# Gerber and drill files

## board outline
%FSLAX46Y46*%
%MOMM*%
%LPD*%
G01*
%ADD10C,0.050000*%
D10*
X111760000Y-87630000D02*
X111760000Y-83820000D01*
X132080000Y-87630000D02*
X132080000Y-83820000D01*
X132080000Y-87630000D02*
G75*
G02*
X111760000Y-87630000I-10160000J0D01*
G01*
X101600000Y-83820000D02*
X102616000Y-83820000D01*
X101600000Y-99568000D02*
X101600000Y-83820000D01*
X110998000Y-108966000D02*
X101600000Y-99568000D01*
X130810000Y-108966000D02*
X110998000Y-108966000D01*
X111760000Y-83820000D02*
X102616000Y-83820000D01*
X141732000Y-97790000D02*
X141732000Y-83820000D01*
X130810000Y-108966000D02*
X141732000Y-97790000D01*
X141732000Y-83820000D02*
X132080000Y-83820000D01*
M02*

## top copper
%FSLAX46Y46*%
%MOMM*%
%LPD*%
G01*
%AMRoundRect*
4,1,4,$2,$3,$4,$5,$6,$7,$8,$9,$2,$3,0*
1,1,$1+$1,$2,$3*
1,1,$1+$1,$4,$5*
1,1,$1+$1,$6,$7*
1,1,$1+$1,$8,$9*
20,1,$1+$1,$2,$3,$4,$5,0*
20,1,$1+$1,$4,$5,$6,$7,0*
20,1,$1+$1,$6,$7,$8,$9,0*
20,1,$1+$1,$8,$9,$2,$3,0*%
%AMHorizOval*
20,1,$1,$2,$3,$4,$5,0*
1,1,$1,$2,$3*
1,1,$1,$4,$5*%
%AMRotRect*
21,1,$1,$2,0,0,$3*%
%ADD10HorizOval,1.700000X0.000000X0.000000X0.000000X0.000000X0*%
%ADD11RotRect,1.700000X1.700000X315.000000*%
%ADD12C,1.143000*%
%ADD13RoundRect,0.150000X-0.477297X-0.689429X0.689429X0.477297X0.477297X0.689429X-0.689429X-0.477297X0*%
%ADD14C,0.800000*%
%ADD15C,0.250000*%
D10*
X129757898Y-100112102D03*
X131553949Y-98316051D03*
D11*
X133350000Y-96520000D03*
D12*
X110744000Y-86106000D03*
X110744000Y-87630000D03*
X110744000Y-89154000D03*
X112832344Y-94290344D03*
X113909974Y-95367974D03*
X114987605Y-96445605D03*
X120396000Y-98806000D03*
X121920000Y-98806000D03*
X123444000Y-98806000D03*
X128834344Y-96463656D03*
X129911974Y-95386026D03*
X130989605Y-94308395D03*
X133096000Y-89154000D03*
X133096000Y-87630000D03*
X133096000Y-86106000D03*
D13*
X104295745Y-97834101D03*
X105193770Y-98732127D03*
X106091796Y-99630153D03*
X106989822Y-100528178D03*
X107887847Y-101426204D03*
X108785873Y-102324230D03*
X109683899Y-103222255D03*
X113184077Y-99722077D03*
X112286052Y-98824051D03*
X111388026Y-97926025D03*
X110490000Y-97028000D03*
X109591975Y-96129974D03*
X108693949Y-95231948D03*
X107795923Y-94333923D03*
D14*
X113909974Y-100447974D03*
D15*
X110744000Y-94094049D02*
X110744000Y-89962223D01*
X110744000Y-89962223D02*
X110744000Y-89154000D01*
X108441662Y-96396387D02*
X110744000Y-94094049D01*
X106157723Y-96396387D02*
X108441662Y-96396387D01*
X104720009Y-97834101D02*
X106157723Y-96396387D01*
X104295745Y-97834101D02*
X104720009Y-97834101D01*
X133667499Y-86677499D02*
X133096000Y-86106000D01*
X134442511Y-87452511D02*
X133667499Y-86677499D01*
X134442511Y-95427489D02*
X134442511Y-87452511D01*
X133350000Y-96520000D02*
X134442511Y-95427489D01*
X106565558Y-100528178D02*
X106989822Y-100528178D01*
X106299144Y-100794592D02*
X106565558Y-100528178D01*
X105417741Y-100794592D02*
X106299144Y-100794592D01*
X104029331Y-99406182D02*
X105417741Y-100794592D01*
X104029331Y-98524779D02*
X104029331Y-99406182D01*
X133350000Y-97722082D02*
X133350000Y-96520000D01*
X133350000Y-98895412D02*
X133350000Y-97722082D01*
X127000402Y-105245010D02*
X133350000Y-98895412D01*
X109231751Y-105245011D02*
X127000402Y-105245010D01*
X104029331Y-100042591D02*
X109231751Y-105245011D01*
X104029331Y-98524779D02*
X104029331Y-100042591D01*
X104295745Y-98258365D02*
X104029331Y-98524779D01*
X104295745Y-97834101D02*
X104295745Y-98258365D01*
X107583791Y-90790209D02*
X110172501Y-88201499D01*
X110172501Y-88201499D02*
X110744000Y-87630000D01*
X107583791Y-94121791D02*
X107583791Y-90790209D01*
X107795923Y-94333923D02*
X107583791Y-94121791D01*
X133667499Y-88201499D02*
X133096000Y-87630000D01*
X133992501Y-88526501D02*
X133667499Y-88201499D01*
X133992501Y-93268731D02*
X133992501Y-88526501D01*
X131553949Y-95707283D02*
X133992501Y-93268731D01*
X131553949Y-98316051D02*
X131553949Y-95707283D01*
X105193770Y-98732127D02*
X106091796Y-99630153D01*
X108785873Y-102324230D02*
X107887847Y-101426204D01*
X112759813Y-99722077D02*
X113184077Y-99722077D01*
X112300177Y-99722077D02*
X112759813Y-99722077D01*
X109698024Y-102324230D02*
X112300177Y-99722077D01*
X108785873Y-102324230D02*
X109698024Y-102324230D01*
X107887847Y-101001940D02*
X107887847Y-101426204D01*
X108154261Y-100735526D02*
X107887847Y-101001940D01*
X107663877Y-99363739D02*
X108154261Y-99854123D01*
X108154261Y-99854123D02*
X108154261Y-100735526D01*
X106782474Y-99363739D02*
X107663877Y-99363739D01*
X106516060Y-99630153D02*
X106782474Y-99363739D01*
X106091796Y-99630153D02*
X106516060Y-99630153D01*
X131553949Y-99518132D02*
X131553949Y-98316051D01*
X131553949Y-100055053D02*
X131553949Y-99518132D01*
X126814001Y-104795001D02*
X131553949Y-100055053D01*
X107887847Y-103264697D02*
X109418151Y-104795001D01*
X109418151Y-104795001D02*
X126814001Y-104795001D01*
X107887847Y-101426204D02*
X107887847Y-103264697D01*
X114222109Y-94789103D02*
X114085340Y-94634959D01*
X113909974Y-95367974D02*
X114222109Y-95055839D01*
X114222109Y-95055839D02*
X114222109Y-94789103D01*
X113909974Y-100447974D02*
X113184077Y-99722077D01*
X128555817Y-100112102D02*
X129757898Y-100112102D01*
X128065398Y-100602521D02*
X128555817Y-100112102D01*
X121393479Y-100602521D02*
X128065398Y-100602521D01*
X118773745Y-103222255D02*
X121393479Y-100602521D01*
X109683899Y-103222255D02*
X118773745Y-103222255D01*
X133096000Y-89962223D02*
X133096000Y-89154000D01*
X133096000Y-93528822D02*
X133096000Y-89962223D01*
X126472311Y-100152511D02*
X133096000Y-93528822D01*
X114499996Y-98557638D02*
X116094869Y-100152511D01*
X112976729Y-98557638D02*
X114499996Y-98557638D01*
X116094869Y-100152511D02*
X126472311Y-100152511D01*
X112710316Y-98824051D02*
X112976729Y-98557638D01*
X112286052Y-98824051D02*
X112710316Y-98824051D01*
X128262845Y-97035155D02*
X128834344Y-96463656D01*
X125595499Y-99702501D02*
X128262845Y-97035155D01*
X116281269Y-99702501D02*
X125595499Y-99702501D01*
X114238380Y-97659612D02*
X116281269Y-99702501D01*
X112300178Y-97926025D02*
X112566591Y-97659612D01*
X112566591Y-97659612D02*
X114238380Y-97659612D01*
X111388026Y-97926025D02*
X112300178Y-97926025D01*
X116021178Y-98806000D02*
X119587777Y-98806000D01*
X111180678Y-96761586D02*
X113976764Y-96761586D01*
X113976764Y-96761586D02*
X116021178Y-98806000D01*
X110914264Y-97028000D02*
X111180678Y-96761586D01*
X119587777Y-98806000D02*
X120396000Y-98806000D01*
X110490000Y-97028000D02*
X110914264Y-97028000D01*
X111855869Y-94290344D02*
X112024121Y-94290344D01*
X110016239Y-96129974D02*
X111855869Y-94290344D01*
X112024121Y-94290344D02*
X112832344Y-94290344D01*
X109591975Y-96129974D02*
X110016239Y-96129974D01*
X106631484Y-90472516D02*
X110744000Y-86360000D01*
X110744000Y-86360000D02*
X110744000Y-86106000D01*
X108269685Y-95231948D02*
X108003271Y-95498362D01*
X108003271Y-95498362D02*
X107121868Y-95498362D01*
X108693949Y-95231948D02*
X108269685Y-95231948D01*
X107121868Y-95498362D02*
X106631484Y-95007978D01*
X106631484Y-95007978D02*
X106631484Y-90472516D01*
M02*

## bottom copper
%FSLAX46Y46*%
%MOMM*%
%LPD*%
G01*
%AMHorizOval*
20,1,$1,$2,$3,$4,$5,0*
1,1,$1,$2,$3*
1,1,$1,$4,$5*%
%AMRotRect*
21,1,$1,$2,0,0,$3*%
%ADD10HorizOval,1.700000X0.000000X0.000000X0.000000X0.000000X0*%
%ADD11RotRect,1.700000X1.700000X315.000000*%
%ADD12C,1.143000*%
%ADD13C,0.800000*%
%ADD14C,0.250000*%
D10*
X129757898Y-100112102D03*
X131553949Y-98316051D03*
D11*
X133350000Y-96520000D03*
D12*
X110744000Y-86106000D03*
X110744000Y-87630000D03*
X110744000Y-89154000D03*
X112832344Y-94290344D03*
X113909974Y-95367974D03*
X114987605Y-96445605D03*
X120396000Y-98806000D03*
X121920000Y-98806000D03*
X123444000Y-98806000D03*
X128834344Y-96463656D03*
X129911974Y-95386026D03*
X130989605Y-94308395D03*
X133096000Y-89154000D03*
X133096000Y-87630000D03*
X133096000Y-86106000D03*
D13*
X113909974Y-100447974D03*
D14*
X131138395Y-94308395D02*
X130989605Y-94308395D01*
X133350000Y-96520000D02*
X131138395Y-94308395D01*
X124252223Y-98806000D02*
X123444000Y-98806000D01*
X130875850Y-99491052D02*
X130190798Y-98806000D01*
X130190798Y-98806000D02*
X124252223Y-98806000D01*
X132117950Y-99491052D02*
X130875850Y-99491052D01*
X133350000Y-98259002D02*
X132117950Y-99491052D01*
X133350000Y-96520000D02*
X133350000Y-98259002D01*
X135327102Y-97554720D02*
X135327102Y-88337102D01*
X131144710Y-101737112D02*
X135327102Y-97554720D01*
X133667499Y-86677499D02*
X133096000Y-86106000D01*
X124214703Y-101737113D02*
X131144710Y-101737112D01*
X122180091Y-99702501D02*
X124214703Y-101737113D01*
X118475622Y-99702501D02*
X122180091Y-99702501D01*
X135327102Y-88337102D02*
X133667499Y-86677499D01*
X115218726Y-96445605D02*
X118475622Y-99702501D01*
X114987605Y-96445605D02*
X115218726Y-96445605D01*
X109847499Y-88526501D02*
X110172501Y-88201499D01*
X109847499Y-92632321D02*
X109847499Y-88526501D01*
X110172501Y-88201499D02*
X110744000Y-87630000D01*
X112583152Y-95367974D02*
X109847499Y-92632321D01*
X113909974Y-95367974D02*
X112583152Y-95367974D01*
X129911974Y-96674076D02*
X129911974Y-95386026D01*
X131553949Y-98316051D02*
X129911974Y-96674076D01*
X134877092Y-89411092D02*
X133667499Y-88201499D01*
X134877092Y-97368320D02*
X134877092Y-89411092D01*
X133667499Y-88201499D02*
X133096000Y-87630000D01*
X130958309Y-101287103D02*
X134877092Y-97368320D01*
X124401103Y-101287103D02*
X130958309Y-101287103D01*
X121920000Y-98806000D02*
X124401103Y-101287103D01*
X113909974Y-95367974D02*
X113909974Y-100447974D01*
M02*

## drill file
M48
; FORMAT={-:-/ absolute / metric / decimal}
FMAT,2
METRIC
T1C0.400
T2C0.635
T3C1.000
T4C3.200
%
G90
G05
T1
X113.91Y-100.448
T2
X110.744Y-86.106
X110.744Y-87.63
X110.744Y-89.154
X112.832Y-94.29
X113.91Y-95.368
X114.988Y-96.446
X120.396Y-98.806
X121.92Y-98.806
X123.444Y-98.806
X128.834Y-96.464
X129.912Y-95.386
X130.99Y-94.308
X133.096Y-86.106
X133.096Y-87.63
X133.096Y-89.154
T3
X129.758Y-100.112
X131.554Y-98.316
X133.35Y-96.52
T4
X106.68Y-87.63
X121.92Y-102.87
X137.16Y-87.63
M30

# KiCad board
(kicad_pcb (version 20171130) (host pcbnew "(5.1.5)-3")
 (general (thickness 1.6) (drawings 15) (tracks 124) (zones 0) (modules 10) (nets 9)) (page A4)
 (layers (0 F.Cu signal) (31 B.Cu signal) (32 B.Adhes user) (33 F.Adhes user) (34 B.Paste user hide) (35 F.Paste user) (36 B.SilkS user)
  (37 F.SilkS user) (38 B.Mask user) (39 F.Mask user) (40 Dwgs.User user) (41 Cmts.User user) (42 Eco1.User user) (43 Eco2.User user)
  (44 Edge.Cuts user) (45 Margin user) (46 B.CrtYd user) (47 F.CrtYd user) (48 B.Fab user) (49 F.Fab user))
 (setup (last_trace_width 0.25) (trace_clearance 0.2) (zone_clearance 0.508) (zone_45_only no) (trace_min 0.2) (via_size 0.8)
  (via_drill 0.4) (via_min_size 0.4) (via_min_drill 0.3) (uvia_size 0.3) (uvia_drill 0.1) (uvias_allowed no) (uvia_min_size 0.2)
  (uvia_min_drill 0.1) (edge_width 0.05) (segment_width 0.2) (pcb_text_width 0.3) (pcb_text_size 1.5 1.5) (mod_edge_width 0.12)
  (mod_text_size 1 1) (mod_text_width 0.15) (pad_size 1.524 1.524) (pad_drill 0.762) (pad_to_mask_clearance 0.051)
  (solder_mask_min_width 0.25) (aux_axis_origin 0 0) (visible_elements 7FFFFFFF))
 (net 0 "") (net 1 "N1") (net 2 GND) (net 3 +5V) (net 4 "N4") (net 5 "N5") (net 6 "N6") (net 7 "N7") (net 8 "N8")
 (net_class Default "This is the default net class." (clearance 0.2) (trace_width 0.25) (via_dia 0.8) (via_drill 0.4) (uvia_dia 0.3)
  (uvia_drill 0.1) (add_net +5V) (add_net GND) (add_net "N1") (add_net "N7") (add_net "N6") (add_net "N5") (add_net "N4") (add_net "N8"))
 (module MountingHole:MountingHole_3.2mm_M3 (layer F.Cu) (at 121.92 102.87)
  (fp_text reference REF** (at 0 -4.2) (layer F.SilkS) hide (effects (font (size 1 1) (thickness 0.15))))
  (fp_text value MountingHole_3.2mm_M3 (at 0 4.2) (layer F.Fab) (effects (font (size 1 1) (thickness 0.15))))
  (pad 1 np_thru_hole circle (at 0 0) (size 3.2 3.2) (drill 3.2) (layers *.Cu *.Mask)))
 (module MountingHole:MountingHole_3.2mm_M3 (layer F.Cu) (at 137.16 87.63)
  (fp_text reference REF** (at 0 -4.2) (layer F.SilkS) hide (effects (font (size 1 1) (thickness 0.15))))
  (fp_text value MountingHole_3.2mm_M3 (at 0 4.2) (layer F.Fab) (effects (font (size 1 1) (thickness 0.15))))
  (pad 1 np_thru_hole circle (at 0 0) (size 3.2 3.2) (drill 3.2) (layers *.Cu *.Mask)))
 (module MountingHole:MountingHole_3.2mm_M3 (layer F.Cu) (at 106.68 87.63)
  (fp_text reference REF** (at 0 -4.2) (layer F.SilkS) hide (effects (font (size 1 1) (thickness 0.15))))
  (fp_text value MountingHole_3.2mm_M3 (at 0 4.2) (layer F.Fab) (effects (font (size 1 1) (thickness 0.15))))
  (pad 1 np_thru_hole circle (at 0 0) (size 3.2 3.2) (drill 3.2) (layers *.Cu *.Mask)))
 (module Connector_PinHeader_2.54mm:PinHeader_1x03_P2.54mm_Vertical (layer F.Cu) (at 133.35 96.52 315)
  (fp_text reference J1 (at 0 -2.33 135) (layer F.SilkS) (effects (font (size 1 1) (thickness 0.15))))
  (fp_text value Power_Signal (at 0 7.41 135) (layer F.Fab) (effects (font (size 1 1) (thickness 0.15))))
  (pad 3 thru_hole oval (at 0 5.08 315) (size 1.7 1.7) (drill 1) (layers *.Cu *.Mask) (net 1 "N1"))
  (pad 2 thru_hole oval (at 0 2.54 315) (size 1.7 1.7) (drill 1) (layers *.Cu *.Mask) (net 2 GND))
  (pad 1 thru_hole rect (at 0 0 315) (size 1.7 1.7) (drill 1) (layers *.Cu *.Mask) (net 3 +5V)))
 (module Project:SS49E (layer F.Cu) (at 110.744 88.9 90)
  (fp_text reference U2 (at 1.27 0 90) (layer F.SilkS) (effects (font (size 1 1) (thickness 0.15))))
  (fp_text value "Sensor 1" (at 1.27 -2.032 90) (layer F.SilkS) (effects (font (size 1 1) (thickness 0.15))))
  (pad 3 thru_hole circle (at 2.794 0 90) (size 1.143 1.143) (drill 0.635) (layers *.Cu *.Mask) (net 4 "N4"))
  (pad 2 thru_hole circle (at 1.27 0 90) (size 1.143 1.143) (drill 0.635) (layers *.Cu *.Mask) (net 2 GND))
  (pad 1 thru_hole circle (at -0.254 0 90) (size 1.143 1.143) (drill 0.635) (layers *.Cu *.Mask) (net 3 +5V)))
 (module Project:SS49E (layer F.Cu) (at 114.808 96.266 135)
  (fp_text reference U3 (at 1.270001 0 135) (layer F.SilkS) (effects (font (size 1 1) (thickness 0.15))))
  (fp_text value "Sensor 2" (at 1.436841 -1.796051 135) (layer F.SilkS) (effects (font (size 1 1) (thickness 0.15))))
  (pad 3 thru_hole circle (at 2.794 0 135) (size 1.143 1.143) (drill 0.635) (layers *.Cu *.Mask) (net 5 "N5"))
  (pad 2 thru_hole circle (at 1.27 0 135) (size 1.143 1.143) (drill 0.635) (layers *.Cu *.Mask) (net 2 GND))
  (pad 1 thru_hole circle (at -0.254 0 135) (size 1.143 1.143) (drill 0.635) (layers *.Cu *.Mask) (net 3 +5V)))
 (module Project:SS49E (layer F.Cu) (at 123.19 98.806 180)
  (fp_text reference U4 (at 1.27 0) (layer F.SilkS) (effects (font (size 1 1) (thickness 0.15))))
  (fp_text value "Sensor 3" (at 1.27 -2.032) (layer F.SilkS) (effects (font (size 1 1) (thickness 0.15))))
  (pad 3 thru_hole circle (at 2.794 0 180) (size 1.143 1.143) (drill 0.635) (layers *.Cu *.Mask) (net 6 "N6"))
  (pad 2 thru_hole circle (at 1.27 0 180) (size 1.143 1.143) (drill 0.635) (layers *.Cu *.Mask) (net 2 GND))
  (pad 1 thru_hole circle (at -0.254 0 180) (size 1.143 1.143) (drill 0.635) (layers *.Cu *.Mask) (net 3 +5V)))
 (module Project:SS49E (layer F.Cu) (at 130.81 94.488 225)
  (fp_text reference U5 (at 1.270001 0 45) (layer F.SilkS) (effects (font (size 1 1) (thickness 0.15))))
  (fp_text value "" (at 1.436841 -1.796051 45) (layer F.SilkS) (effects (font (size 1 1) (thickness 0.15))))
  (pad 3 thru_hole circle (at 2.794 0 225) (size 1.143 1.143) (drill 0.635) (layers *.Cu *.Mask) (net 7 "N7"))
  (pad 2 thru_hole circle (at 1.27 0 225) (size 1.143 1.143) (drill 0.635) (layers *.Cu *.Mask) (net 2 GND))
  (pad 1 thru_hole circle (at -0.254 0 225) (size 1.143 1.143) (drill 0.635) (layers *.Cu *.Mask) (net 3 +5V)))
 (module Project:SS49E (layer F.Cu) (at 133.096 86.36 270)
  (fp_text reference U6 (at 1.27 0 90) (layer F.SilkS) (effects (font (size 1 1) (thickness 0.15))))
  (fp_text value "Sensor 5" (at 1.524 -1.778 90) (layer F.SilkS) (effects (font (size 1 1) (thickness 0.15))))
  (pad 3 thru_hole circle (at 2.794 0 270) (size 1.143 1.143) (drill 0.635) (layers *.Cu *.Mask) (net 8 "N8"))
  (pad 2 thru_hole circle (at 1.27 0 270) (size 1.143 1.143) (drill 0.635) (layers *.Cu *.Mask) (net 2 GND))
  (pad 1 thru_hole circle (at -0.254 0 270) (size 1.143 1.143) (drill 0.635) (layers *.Cu *.Mask) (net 3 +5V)))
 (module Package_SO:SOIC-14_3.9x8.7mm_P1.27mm (layer F.Cu) (at 108.739911 98.778089 45)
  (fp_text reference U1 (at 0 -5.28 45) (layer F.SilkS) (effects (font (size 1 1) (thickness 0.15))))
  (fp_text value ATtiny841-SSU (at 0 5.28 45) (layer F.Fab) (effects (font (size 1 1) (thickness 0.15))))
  (pad 1 smd roundrect (at -2.475 -3.81 45) (size 1.95 0.6) (layers F.Cu F.Paste F.Mask) (roundrect_rratio 0.25) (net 3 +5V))
  (pad 2 smd roundrect (at -2.475 -2.54 45) (size 1.95 0.6) (layers F.Cu F.Paste F.Mask) (roundrect_rratio 0.25) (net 2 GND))
  (pad 3 smd roundrect (at -2.475 -1.27 45) (size 1.95 0.6) (layers F.Cu F.Paste F.Mask) (roundrect_rratio 0.25) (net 2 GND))
  (pad 4 smd roundrect (at -2.475 0 45) (size 1.95 0.6) (layers F.Cu F.Paste F.Mask) (roundrect_rratio 0.25) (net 3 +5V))
  (pad 5 smd roundrect (at -2.475 1.27 45) (size 1.95 0.6) (layers F.Cu F.Paste F.Mask) (roundrect_rratio 0.25) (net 2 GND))
  (pad 6 smd roundrect (at -2.475 2.54 45) (size 1.95 0.6) (layers F.Cu F.Paste F.Mask) (roundrect_rratio 0.25) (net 2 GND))
  (pad 7 smd roundrect (at -2.475 3.81 45) (size 1.95 0.6) (layers F.Cu F.Paste F.Mask) (roundrect_rratio 0.25) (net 1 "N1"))
  (pad 8 smd roundrect (at 2.475 3.81 45) (size 1.95 0.6) (layers F.Cu F.Paste F.Mask) (roundrect_rratio 0.25) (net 2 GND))
  (pad 9 smd roundrect (at 2.475 2.54 45) (size 1.95 0.6) (layers F.Cu F.Paste F.Mask) (roundrect_rratio 0.25) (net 8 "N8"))
  (pad 10 smd roundrect (at 2.475 1.27 45) (size 1.95 0.6) (layers F.Cu F.Paste F.Mask) (roundrect_rratio 0.25) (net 7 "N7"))
  (pad 11 smd roundrect (at 2.475 0 45) (size 1.95 0.6) (layers F.Cu F.Paste F.Mask) (roundrect_rratio 0.25) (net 6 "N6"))
  (pad 12 smd roundrect (at 2.475 -1.27 45) (size 1.95 0.6) (layers F.Cu F.Paste F.Mask) (roundrect_rratio 0.25) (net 5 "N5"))
  (pad 13 smd roundrect (at 2.475 -2.54 45) (size 1.95 0.6) (layers F.Cu F.Paste F.Mask) (roundrect_rratio 0.25) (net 4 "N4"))
  (pad 14 smd roundrect (at 2.475 -3.81 45) (size 1.95 0.6) (layers F.Cu F.Paste F.Mask) (roundrect_rratio 0.25) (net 2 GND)))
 (gr_line (start 111.76 87.63) (end 111.76 83.82) (layer Edge.Cuts) (width 0.05))
 (gr_line (start 132.08 87.63) (end 132.08 83.82) (layer Edge.Cuts) (width 0.05))
 (gr_arc (start 121.92 87.63) (end 111.76 87.63) (angle -180) (layer Edge.Cuts) (width 0.05))
 (gr_line (start 101.6 83.82) (end 102.616 83.82) (layer Edge.Cuts) (width 0.05))
 (gr_line (start 101.6 99.568) (end 101.6 83.82) (layer Edge.Cuts) (width 0.05))
 (gr_line (start 110.998 108.966) (end 101.6 99.568) (layer Edge.Cuts) (width 0.05))
 (gr_line (start 130.81 108.966) (end 110.998 108.966) (layer Edge.Cuts) (width 0.05))
 (gr_line (start 111.76 83.82) (end 102.616 83.82) (layer Edge.Cuts) (width 0.05))
 (gr_line (start 141.732 97.79) (end 141.732 83.82) (layer Edge.Cuts) (width 0.05))
 (gr_line (start 130.81 108.966) (end 141.732 97.79) (layer Edge.Cuts) (width 0.05))
 (gr_line (start 141.732 83.82) (end 132.08 83.82) (layer Edge.Cuts) (width 0.05))
 (segment (start 110.744 94.094049) (end 110.744 89.962223) (width 0.25) (layer F.Cu) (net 3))
 (segment (start 110.744 89.962223) (end 110.744 89.154) (width 0.25) (layer F.Cu) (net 3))
 (segment (start 108.441662 96.396387) (end 110.744 94.094049) (width 0.25) (layer F.Cu) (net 3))
 (segment (start 106.157723 96.396387) (end 108.441662 96.396387) (width 0.25) (layer F.Cu) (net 3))
 (segment (start 104.720009 97.834101) (end 106.157723 96.396387) (width 0.25) (layer F.Cu) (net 3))
 (segment (start 104.295745 97.834101) (end 104.720009 97.834101) (width 0.25) (layer F.Cu) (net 3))
 (segment (start 133.667499 86.677499) (end 133.096 86.106) (width 0.25) (layer F.Cu) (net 3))
 (segment (start 134.442511 87.452511) (end 133.667499 86.677499) (width 0.25) (layer F.Cu) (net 3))
 (segment (start 134.442511 95.427489) (end 134.442511 87.452511) (width 0.25) (layer F.Cu) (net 3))
 (segment (start 133.35 96.52) (end 134.442511 95.427489) (width 0.25) (layer F.Cu) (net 3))
 (segment (start 106.565558 100.528178) (end 106.989822 100.528178) (width 0.25) (layer F.Cu) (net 3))
 (segment (start 106.299144 100.794592) (end 106.565558 100.528178) (width 0.25) (layer F.Cu) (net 3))
 (segment (start 105.417741 100.794592) (end 106.299144 100.794592) (width 0.25) (layer F.Cu) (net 3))
 (segment (start 104.029331 99.406182) (end 105.417741 100.794592) (width 0.25) (layer F.Cu) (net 3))
 (segment (start 104.029331 98.524779) (end 104.029331 99.406182) (width 0.25) (layer F.Cu) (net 3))
 (segment (start 131.138395 94.308395) (end 130.989605 94.308395) (width 0.25) (layer B.Cu) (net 3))
 (segment (start 133.35 96.52) (end 131.138395 94.308395) (width 0.25) (layer B.Cu) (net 3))
 (segment (start 124.252223 98.806) (end 123.444 98.806) (width 0.25) (layer B.Cu) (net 3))
 (segment (start 130.87585 99.491052) (end 130.190798 98.806) (width 0.25) (layer B.Cu) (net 3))
 (segment (start 130.190798 98.806) (end 124.252223 98.806) (width 0.25) (layer B.Cu) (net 3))
 (segment (start 132.11795 99.491052) (end 130.87585 99.491052) (width 0.25) (layer B.Cu) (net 3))
 (segment (start 133.35 98.259002) (end 132.11795 99.491052) (width 0.25) (layer B.Cu) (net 3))
 (segment (start 133.35 96.52) (end 133.35 98.259002) (width 0.25) (layer B.Cu) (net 3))
 (segment (start 135.327102 97.55472) (end 135.327102 88.337102) (width 0.25) (layer B.Cu) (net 3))
 (segment (start 131.14471 101.737112) (end 135.327102 97.55472) (width 0.25) (layer B.Cu) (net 3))
 (segment (start 133.667499 86.677499) (end 133.096 86.106) (width 0.25) (layer B.Cu) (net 3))
 (segment (start 124.214703 101.737113) (end 131.14471 101.737112) (width 0.25) (layer B.Cu) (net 3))
 (segment (start 122.180091 99.702501) (end 124.214703 101.737113) (width 0.25) (layer B.Cu) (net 3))
 (segment (start 118.475622 99.702501) (end 122.180091 99.702501) (width 0.25) (layer B.Cu) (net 3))
 (segment (start 135.327102 88.337102) (end 133.667499 86.677499) (width 0.25) (layer B.Cu) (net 3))
 (segment (start 115.218726 96.445605) (end 118.475622 99.702501) (width 0.25) (layer B.Cu) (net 3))
 (segment (start 114.987605 96.445605) (end 115.218726 96.445605) (width 0.25) (layer B.Cu) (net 3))
 (segment (start 133.35 97.722082) (end 133.35 96.52) (width 0.25) (layer F.Cu) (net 3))
 (segment (start 133.35 98.895412) (end 133.35 97.722082) (width 0.25) (layer F.Cu) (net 3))
 (segment (start 127.000402 105.24501) (end 133.35 98.895412) (width 0.25) (layer F.Cu) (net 3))
 (segment (start 109.231751 105.245011) (end 127.000402 105.24501) (width 0.25) (layer F.Cu) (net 3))
 (segment (start 104.029331 100.042591) (end 109.231751 105.245011) (width 0.25) (layer F.Cu) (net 3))
 (segment (start 104.029331 98.524779) (end 104.029331 100.042591) (width 0.25) (layer F.Cu) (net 3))
 (segment (start 104.295745 98.258365) (end 104.029331 98.524779) (width 0.25) (layer F.Cu) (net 3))
 (segment (start 104.295745 97.834101) (end 104.295745 98.258365) (width 0.25) (layer F.Cu) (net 3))
 (segment (start 107.583791 90.790209) (end 110.172501 88.201499) (width 0.25) (layer F.Cu) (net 2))
 (segment (start 110.172501 88.201499) (end 110.744 87.63) (width 0.25) (layer F.Cu) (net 2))
 (segment (start 107.583791 94.121791) (end 107.583791 90.790209) (width 0.25) (layer F.Cu) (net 2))
 (segment (start 107.795923 94.333923) (end 107.583791 94.121791) (width 0.25) (layer F.Cu) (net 2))
 (segment (start 133.667499 88.201499) (end 133.096 87.63) (width 0.25) (layer F.Cu) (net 2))
 (segment (start 133.992501 88.526501) (end 133.667499 88.201499) (width 0.25) (layer F.Cu) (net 2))
 (segment (start 133.992501 93.268731) (end 133.992501 88.526501) (width 0.25) (layer F.Cu) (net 2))
 (segment (start 131.553949 95.707283) (end 133.992501 93.268731) (width 0.25) (layer F.Cu) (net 2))
 (segment (start 131.553949 98.316051) (end 131.553949 95.707283) (width 0.25) (layer F.Cu) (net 2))
 (segment (start 105.19377 98.732127) (end 106.091796 99.630153) (width 0.25) (layer F.Cu) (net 2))
 (segment (start 108.785873 102.32423) (end 107.887847 101.426204) (width 0.25) (layer F.Cu) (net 2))
 (segment (start 112.759813 99.722077) (end 113.184077 99.722077) (width 0.25) (layer F.Cu) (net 2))
 (segment (start 112.300177 99.722077) (end 112.759813 99.722077) (width 0.25) (layer F.Cu) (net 2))
 (segment (start 109.698024 102.32423) (end 112.300177 99.722077) (width 0.25) (layer F.Cu) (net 2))
 (segment (start 108.785873 102.32423) (end 109.698024 102.32423) (width 0.25) (layer F.Cu) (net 2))
 (segment (start 107.887847 101.00194) (end 107.887847 101.426204) (width 0.25) (layer F.Cu) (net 2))
 (segment (start 108.154261 100.735526) (end 107.887847 101.00194) (width 0.25) (layer F.Cu) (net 2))
 (segment (start 107.663877 99.363739) (end 108.154261 99.854123) (width 0.25) (layer F.Cu) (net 2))
 (segment (start 108.154261 99.854123) (end 108.154261 100.735526) (width 0.25) (layer F.Cu) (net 2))
 (segment (start 106.782474 99.363739) (end 107.663877 99.363739) (width 0.25) (layer F.Cu) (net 2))
 (segment (start 106.51606 99.630153) (end 106.782474 99.363739) (width 0.25) (layer F.Cu) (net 2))
 (segment (start 106.091796 99.630153) (end 106.51606 99.630153) (width 0.25) (layer F.Cu) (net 2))
 (segment (start 131.553949 99.518132) (end 131.553949 98.316051) (width 0.25) (layer F.Cu) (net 2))
 (segment (start 131.553949 100.055053) (end 131.553949 99.518132) (width 0.25) (layer F.Cu) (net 2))
 (segment (start 126.814001 104.795001) (end 131.553949 100.055053) (width 0.25) (layer F.Cu) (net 2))
 (segment (start 107.887847 103.264697) (end 109.418151 104.795001) (width 0.25) (layer F.Cu) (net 2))
 (segment (start 109.418151 104.795001) (end 126.814001 104.795001) (width 0.25) (layer F.Cu) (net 2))
 (segment (start 107.887847 101.426204) (end 107.887847 103.264697) (width 0.25) (layer F.Cu) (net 2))
 (segment (start 109.847499 88.526501) (end 110.172501 88.201499) (width 0.25) (layer B.Cu) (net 2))
 (segment (start 109.847499 92.632321) (end 109.847499 88.526501) (width 0.25) (layer B.Cu) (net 2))
 (segment (start 110.172501 88.201499) (end 110.744 87.63) (width 0.25) (layer B.Cu) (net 2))
 (segment (start 112.583152 95.367974) (end 109.847499 92.632321) (width 0.25) (layer B.Cu) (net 2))
 (segment (start 113.909974 95.367974) (end 112.583152 95.367974) (width 0.25) (layer B.Cu) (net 2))
 (segment (start 129.911974 96.674076) (end 129.911974 95.386026) (width 0.25) (layer B.Cu) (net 2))
 (segment (start 131.553949 98.316051) (end 129.911974 96.674076) (width 0.25) (layer B.Cu) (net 2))
 (segment (start 114.222109 94.789103) (end 114.08534 94.634959) (width 0.25) (layer F.Cu) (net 2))
 (segment (start 113.909974 95.367974) (end 114.222109 95.055839) (width 0.25) (layer F.Cu) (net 2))
 (segment (start 114.222109 95.055839) (end 114.222109 94.789103) (width 0.25) (layer F.Cu) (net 2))
 (segment (start 134.877092 89.411092) (end 133.667499 88.201499) (width 0.25) (layer B.Cu) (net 2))
 (segment (start 134.877092 97.36832) (end 134.877092 89.411092) (width 0.25) (layer B.Cu) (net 2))
 (segment (start 133.667499 88.201499) (end 133.096 87.63) (width 0.25) (layer B.Cu) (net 2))
 (segment (start 130.958309 101.287103) (end 134.877092 97.36832) (width 0.25) (layer B.Cu) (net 2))
 (segment (start 124.401103 101.287103) (end 130.958309 101.287103) (width 0.25) (layer B.Cu) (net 2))
 (segment (start 121.92 98.806) (end 124.401103 101.287103) (width 0.25) (layer B.Cu) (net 2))
 (segment (start 113.909974 95.367974) (end 113.909974 100.447974) (width 0.25) (layer B.Cu) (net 2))
 (via (at 113.909974 100.447974) (size 0.8) (drill 0.4) (layers F.Cu B.Cu) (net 2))
 (segment (start 113.909974 100.447974) (end 113.184077 99.722077) (width 0.25) (layer F.Cu) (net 2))
 (segment (start 128.555817 100.112102) (end 129.757898 100.112102) (width 0.25) (layer F.Cu) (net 1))
 (segment (start 128.065398 100.602521) (end 128.555817 100.112102) (width 0.25) (layer F.Cu) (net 1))
 (segment (start 121.393479 100.602521) (end 128.065398 100.602521) (width 0.25) (layer F.Cu) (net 1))
 (segment (start 118.773745 103.222255) (end 121.393479 100.602521) (width 0.25) (layer F.Cu) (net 1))
 (segment (start 109.683899 103.222255) (end 118.773745 103.222255) (width 0.25) (layer F.Cu) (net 1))
 (segment (start 133.096 89.962223) (end 133.096 89.154) (width 0.25) (layer F.Cu) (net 8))
 (segment (start 133.096 93.528822) (end 133.096 89.962223) (width 0.25) (layer F.Cu) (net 8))
 (segment (start 126.472311 100.152511) (end 133.096 93.528822) (width 0.25) (layer F.Cu) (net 8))
 (segment (start 114.499996 98.557638) (end 116.094869 100.152511) (width 0.25) (layer F.Cu) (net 8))
 (segment (start 112.976729 98.557638) (end 114.499996 98.557638) (width 0.25) (layer F.Cu) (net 8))
 (segment (start 116.094869 100.152511) (end 126.472311 100.152511) (width 0.25) (layer F.Cu) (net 8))
 (segment (start 112.710316 98.824051) (end 112.976729 98.557638) (width 0.25) (layer F.Cu) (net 8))
 (segment (start 112.286052 98.824051) (end 112.710316 98.824051) (width 0.25) (layer F.Cu) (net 8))
 (segment (start 128.262845 97.035155) (end 128.834344 96.463656) (width 0.25) (layer F.Cu) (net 7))
 (segment (start 125.595499 99.702501) (end 128.262845 97.035155) (width 0.25) (layer F.Cu) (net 7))
 (segment (start 116.281269 99.702501) (end 125.595499 99.702501) (width 0.25) (layer F.Cu) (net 7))
 (segment (start 114.23838 97.659612) (end 116.281269 99.702501) (width 0.25) (layer F.Cu) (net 7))
 (segment (start 112.300178 97.926025) (end 112.566591 97.659612) (width 0.25) (layer F.Cu) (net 7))
 (segment (start 112.566591 97.659612) (end 114.23838 97.659612) (width 0.25) (layer F.Cu) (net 7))
 (segment (start 111.388026 97.926025) (end 112.300178 97.926025) (width 0.25) (layer F.Cu) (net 7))
 (segment (start 116.021178 98.806) (end 119.587777 98.806) (width 0.25) (layer F.Cu) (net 6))
 (segment (start 111.180678 96.761586) (end 113.976764 96.761586) (width 0.25) (layer F.Cu) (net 6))
 (segment (start 113.976764 96.761586) (end 116.021178 98.806) (width 0.25) (layer F.Cu) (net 6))
 (segment (start 110.914264 97.028) (end 111.180678 96.761586) (width 0.25) (layer F.Cu) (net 6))
 (segment (start 119.587777 98.806) (end 120.396 98.806) (width 0.25) (layer F.Cu) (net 6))
 (segment (start 110.49 97.028) (end 110.914264 97.028) (width 0.25) (layer F.Cu) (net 6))
 (segment (start 111.855869 94.290344) (end 112.024121 94.290344) (width 0.25) (layer F.Cu) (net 5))
 (segment (start 110.016239 96.129974) (end 111.855869 94.290344) (width 0.25) (layer F.Cu) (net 5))
 (segment (start 112.024121 94.290344) (end 112.832344 94.290344) (width 0.25) (layer F.Cu) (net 5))
 (segment (start 109.591975 96.129974) (end 110.016239 96.129974) (width 0.25) (layer F.Cu) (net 5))
 (segment (start 106.631484 90.472516) (end 110.744 86.36) (width 0.25) (layer F.Cu) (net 4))
 (segment (start 110.744 86.36) (end 110.744 86.106) (width 0.25) (layer F.Cu) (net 4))
 (segment (start 108.269685 95.231948) (end 108.003271 95.498362) (width 0.25) (layer F.Cu) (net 4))
 (segment (start 108.003271 95.498362) (end 107.121868 95.498362) (width 0.25) (layer F.Cu) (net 4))
 (segment (start 108.693949 95.231948) (end 108.269685 95.231948) (width 0.25) (layer F.Cu) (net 4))
 (segment (start 107.121868 95.498362) (end 106.631484 95.007978) (width 0.25) (layer F.Cu) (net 4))
 (segment (start 106.631484 95.007978) (end 106.631484 90.472516) (width 0.25) (layer F.Cu) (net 4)))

